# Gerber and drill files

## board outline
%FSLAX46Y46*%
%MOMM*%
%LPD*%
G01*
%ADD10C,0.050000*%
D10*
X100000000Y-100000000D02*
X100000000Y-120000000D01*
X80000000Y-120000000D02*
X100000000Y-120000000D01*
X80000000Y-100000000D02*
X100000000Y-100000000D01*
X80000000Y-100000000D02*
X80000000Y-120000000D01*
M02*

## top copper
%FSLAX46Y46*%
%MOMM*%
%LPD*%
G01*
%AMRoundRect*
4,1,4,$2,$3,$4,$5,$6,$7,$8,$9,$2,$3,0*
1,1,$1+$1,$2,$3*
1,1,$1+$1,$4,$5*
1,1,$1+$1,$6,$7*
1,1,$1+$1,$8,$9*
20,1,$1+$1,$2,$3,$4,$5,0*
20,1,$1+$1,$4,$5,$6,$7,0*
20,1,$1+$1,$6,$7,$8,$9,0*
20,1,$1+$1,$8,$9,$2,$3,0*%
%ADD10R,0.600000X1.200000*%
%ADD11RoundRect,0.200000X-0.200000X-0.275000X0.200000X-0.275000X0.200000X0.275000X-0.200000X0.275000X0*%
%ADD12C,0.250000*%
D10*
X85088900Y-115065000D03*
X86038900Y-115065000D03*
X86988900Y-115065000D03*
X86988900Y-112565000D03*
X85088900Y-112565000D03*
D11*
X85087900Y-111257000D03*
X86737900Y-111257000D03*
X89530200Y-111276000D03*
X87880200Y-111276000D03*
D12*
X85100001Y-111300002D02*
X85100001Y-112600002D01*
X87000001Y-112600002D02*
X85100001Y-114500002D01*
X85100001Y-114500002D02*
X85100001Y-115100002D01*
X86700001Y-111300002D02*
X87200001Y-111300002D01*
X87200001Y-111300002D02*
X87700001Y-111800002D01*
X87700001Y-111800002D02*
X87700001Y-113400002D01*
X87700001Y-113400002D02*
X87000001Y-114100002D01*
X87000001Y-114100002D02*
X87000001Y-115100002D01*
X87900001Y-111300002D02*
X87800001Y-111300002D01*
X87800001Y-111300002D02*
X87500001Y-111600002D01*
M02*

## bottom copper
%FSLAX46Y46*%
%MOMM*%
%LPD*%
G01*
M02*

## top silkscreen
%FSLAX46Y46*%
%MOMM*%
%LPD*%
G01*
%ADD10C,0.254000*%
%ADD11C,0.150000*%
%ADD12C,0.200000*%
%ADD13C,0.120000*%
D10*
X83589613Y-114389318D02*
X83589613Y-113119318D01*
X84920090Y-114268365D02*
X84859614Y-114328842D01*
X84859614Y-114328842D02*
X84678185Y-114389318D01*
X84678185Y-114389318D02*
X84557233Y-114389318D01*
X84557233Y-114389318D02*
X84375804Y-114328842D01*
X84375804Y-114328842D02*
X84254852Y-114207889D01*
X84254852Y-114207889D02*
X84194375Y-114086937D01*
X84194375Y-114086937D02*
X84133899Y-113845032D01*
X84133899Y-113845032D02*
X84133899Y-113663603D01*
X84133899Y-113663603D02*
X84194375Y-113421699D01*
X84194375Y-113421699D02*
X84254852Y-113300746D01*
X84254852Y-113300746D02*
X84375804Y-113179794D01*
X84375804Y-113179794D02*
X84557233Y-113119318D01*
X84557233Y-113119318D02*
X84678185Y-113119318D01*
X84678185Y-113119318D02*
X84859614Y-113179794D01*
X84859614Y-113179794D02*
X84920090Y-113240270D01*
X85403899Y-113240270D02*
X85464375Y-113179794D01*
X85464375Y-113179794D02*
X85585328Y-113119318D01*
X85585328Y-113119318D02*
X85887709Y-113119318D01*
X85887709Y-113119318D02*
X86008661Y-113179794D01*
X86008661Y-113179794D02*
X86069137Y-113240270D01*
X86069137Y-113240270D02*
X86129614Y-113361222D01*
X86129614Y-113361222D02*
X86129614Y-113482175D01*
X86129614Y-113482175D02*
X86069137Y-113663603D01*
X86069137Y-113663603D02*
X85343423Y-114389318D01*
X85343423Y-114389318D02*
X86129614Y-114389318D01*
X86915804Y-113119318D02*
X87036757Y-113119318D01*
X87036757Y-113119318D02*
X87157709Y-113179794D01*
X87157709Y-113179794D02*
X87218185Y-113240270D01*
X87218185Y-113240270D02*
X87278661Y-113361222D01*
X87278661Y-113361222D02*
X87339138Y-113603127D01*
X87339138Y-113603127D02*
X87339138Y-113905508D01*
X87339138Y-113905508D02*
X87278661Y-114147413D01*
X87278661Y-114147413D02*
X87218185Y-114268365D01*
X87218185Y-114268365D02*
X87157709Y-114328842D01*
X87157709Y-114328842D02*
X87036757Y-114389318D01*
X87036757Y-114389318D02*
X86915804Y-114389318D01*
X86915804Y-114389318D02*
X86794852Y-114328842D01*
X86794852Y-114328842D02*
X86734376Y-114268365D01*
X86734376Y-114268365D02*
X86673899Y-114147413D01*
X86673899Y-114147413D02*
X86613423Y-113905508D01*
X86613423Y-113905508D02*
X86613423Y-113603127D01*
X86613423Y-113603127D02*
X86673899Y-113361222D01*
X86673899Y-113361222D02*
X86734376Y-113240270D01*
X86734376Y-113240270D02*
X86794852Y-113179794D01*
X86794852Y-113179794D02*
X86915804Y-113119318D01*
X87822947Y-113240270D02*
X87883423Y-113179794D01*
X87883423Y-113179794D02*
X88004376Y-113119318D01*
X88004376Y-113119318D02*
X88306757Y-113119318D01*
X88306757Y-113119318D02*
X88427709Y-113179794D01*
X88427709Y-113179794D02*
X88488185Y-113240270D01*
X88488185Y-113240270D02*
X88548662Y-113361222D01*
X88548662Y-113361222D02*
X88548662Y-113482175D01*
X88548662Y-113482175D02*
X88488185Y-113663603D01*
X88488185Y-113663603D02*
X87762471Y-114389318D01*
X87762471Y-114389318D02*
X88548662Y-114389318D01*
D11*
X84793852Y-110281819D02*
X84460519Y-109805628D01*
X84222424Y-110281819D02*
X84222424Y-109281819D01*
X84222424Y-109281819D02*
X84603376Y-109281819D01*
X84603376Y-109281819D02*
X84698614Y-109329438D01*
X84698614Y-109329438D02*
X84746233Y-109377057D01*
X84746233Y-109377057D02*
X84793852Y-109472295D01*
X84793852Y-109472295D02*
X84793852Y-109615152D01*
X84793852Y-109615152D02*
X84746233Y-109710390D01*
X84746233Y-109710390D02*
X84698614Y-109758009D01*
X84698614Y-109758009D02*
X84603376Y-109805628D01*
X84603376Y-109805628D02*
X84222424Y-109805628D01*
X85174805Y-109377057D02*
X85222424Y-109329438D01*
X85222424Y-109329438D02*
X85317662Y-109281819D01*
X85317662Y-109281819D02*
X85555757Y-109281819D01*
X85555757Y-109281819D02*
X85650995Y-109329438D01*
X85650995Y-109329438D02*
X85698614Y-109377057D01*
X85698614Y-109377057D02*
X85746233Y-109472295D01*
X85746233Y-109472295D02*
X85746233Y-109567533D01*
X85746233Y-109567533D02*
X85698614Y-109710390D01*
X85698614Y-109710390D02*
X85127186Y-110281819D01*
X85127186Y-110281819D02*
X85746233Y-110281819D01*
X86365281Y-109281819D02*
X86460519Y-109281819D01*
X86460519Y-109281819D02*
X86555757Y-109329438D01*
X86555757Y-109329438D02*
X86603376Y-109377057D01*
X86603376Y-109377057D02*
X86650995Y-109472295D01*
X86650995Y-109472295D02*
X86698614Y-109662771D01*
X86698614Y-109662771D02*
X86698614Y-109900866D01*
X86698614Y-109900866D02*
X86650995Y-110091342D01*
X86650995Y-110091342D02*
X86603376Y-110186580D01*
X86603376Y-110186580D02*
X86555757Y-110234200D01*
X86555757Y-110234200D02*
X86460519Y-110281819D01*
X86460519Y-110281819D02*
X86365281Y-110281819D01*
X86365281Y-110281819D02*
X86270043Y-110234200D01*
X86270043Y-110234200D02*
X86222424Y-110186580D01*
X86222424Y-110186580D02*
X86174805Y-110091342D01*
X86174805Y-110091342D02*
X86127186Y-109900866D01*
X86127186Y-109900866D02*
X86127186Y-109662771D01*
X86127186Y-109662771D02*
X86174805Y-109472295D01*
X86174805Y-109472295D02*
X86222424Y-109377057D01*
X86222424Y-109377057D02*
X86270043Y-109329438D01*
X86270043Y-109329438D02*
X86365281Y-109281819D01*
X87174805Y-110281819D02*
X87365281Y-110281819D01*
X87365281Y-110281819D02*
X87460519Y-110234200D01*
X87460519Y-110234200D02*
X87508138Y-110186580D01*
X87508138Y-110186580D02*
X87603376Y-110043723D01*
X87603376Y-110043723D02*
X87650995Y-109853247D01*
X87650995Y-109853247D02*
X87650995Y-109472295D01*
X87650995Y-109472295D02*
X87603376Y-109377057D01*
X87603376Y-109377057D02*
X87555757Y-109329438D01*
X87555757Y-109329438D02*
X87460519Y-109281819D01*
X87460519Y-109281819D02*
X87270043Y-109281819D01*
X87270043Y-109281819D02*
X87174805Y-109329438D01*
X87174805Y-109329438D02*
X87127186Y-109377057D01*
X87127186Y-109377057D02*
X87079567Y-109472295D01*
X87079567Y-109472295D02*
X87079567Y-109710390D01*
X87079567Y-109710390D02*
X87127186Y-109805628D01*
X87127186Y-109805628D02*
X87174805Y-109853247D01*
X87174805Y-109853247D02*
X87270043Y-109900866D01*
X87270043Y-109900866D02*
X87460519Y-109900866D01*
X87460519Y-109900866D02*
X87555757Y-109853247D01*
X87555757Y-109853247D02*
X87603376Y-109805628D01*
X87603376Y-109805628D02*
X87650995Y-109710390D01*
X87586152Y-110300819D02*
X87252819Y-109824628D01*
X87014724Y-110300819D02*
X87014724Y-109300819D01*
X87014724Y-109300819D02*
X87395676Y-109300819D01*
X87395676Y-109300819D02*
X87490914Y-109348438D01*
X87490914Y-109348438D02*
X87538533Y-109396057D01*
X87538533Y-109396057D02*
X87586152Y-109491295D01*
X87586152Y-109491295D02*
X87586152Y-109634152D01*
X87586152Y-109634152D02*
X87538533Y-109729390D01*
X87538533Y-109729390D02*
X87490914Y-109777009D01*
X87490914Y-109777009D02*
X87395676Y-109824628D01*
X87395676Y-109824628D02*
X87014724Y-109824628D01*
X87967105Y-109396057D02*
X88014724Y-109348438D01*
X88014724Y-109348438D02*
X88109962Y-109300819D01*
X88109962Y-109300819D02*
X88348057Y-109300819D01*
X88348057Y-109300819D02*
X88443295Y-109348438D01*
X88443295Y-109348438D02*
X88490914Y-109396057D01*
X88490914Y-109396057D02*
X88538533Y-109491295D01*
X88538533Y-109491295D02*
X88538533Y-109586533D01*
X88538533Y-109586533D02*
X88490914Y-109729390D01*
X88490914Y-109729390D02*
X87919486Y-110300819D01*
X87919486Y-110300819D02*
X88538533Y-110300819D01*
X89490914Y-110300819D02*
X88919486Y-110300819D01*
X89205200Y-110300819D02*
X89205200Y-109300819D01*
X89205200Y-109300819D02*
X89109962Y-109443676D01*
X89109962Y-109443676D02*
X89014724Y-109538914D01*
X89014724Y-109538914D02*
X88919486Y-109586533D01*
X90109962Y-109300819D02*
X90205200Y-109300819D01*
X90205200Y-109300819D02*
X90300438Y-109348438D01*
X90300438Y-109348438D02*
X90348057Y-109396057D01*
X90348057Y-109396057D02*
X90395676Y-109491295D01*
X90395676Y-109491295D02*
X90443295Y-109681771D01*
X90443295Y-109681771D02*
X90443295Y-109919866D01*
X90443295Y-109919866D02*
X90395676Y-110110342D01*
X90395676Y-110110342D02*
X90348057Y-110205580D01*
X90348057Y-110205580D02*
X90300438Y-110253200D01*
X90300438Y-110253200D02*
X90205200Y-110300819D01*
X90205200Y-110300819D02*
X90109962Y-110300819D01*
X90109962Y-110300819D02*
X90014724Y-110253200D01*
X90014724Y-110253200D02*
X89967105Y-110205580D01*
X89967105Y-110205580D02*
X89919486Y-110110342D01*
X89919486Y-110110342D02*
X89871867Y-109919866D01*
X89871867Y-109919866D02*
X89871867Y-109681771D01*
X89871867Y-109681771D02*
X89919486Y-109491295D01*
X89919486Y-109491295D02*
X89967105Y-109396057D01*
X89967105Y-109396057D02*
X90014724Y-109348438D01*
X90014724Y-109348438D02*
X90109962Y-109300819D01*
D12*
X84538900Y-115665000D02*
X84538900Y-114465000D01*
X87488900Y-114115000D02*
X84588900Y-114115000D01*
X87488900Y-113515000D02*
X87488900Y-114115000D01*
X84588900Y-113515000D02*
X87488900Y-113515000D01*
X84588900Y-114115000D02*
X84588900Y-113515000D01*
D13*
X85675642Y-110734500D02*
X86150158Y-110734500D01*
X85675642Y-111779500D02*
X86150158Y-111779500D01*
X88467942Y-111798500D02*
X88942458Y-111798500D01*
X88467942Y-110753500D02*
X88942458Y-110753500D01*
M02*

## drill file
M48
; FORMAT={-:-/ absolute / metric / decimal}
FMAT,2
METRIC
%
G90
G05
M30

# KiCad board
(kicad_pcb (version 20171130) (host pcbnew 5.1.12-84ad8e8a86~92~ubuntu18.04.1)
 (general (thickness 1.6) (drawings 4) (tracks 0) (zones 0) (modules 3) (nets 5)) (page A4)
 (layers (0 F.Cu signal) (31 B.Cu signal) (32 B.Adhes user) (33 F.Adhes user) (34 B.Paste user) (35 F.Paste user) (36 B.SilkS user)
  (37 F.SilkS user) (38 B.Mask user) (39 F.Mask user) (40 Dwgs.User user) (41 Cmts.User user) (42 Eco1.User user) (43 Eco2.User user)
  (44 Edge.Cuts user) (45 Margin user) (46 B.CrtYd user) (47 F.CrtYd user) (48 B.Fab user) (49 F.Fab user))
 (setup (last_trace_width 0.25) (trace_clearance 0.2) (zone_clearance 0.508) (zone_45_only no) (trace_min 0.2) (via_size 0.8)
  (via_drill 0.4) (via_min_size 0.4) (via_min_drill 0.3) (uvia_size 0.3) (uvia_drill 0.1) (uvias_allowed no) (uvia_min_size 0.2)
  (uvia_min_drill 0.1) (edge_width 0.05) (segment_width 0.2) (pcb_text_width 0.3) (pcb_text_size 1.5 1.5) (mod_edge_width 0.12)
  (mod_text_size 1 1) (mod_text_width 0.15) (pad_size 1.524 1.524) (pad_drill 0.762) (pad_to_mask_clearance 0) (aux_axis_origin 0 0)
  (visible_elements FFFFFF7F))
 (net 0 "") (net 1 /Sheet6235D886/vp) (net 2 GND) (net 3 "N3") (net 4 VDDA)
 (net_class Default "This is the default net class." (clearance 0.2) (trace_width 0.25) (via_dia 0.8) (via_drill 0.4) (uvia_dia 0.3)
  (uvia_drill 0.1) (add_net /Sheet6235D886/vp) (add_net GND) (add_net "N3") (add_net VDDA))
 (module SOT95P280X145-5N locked (layer F.Cu) (at 86.038900 113.815000 90.000000)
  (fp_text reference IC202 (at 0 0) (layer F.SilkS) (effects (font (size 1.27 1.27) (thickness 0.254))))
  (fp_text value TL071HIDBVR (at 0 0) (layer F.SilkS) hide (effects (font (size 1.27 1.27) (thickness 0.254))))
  (fp_line (start -1.85 -1.5) (end -0.65 -1.5) (layer F.SilkS) (width 0.2))
  (fp_line (start -0.3 1.45) (end -0.3 -1.45) (layer F.SilkS) (width 0.2))
  (fp_line (start 0.3 1.45) (end -0.3 1.45) (layer F.SilkS) (width 0.2))
  (fp_line (start 0.3 -1.45) (end 0.3 1.45) (layer F.SilkS) (width 0.2))
  (fp_line (start -0.3 -1.45) (end 0.3 -1.45) (layer F.SilkS) (width 0.2))
  (pad 1 smd rect (at -1.25 -0.95 180.000000) (size 0.6 1.2) (layers F.Cu F.Mask F.Paste) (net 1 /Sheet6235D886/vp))
  (pad 2 smd rect (at -1.25 0 180.000000) (size 0.6 1.2) (layers F.Cu F.Mask F.Paste) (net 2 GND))
  (pad 3 smd rect (at -1.25 0.95 180.000000) (size 0.6 1.2) (layers F.Cu F.Mask F.Paste) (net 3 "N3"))
  (pad 4 smd rect (at 1.25 0.95 180.000000) (size 0.6 1.2) (layers F.Cu F.Mask F.Paste) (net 1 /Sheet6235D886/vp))
  (pad 5 smd rect (at 1.25 -0.95 180.000000) (size 0.6 1.2) (layers F.Cu F.Mask F.Paste) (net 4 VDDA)))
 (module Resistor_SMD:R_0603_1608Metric (layer F.Cu) (at 85.912900 111.257000)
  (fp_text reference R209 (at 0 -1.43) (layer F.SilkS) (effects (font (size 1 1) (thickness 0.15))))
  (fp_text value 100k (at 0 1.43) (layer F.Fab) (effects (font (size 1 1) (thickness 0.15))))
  (fp_line (start -0.237258 -0.5225) (end 0.237258 -0.5225) (layer F.SilkS) (width 0.12))
  (fp_line (start -0.237258 0.5225) (end 0.237258 0.5225) (layer F.SilkS) (width 0.12))
  (pad 1 smd roundrect (at -0.825 0) (size 0.8 0.95) (layers F.Cu F.Mask F.Paste) (roundrect_rratio 0.25) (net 4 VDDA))
  (pad 2 smd roundrect (at 0.825 0) (size 0.8 0.95) (layers F.Cu F.Mask F.Paste) (roundrect_rratio 0.25) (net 3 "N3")))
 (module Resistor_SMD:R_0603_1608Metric (layer F.Cu) (at 88.705200 111.276000)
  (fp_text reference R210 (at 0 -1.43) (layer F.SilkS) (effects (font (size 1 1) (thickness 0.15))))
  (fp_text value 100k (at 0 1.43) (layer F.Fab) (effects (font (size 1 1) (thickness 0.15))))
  (fp_line (start -0.237258 0.5225) (end 0.237258 0.5225) (layer F.SilkS) (width 0.12))
  (fp_line (start -0.237258 -0.5225) (end 0.237258 -0.5225) (layer F.SilkS) (width 0.12))
  (pad 2 smd roundrect (at 0.825 0) (size 0.8 0.95) (layers F.Cu F.Mask F.Paste) (roundrect_rratio 0.25) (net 2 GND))
  (pad 1 smd roundrect (at -0.825 0) (size 0.8 0.95) (layers F.Cu F.Mask F.Paste) (roundrect_rratio 0.25) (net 3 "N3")))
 (gr_line (start 100 100) (end 100 120) (layer Edge.Cuts) (width 0.05))
 (gr_line (start 80 120) (end 100 120) (layer Edge.Cuts) (width 0.05))
 (gr_line (start 80 100) (end 100 100) (layer Edge.Cuts) (width 0.05))
 (gr_line (start 80 100) (end 80 120) (layer Edge.Cuts) (width 0.05))
 (segment (start 85.100001 111.300002) (end 85.100001 112.600002) (width 0.250000) (layer F.Cu) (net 4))
 (segment (start 87.000001 112.600002) (end 85.100001 114.500002) (width 0.250000) (layer F.Cu) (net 1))
 (segment (start 85.100001 114.500002) (end 85.100001 115.100002) (width 0.250000) (layer F.Cu) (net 1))
 (segment (start 86.700001 111.300002) (end 87.200001 111.300002) (width 0.250000) (layer F.Cu) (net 3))
 (segment (start 87.200001 111.300002) (end 87.700001 111.800002) (width 0.250000) (layer F.Cu) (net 3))
 (segment (start 87.700001 111.800002) (end 87.700001 113.400002) (width 0.250000) (layer F.Cu) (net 3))
 (segment (start 87.700001 113.400002) (end 87.000001 114.100002) (width 0.250000) (layer F.Cu) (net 3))
 (segment (start 87.000001 114.100002) (end 87.000001 115.100002) (width 0.250000) (layer F.Cu) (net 3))
 (segment (start 87.900001 111.300002) (end 87.800001 111.300002) (width 0.250000) (layer F.Cu) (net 3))
 (segment (start 87.800001 111.300002) (end 87.500001 111.600002) (width 0.250000) (layer F.Cu) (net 3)))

